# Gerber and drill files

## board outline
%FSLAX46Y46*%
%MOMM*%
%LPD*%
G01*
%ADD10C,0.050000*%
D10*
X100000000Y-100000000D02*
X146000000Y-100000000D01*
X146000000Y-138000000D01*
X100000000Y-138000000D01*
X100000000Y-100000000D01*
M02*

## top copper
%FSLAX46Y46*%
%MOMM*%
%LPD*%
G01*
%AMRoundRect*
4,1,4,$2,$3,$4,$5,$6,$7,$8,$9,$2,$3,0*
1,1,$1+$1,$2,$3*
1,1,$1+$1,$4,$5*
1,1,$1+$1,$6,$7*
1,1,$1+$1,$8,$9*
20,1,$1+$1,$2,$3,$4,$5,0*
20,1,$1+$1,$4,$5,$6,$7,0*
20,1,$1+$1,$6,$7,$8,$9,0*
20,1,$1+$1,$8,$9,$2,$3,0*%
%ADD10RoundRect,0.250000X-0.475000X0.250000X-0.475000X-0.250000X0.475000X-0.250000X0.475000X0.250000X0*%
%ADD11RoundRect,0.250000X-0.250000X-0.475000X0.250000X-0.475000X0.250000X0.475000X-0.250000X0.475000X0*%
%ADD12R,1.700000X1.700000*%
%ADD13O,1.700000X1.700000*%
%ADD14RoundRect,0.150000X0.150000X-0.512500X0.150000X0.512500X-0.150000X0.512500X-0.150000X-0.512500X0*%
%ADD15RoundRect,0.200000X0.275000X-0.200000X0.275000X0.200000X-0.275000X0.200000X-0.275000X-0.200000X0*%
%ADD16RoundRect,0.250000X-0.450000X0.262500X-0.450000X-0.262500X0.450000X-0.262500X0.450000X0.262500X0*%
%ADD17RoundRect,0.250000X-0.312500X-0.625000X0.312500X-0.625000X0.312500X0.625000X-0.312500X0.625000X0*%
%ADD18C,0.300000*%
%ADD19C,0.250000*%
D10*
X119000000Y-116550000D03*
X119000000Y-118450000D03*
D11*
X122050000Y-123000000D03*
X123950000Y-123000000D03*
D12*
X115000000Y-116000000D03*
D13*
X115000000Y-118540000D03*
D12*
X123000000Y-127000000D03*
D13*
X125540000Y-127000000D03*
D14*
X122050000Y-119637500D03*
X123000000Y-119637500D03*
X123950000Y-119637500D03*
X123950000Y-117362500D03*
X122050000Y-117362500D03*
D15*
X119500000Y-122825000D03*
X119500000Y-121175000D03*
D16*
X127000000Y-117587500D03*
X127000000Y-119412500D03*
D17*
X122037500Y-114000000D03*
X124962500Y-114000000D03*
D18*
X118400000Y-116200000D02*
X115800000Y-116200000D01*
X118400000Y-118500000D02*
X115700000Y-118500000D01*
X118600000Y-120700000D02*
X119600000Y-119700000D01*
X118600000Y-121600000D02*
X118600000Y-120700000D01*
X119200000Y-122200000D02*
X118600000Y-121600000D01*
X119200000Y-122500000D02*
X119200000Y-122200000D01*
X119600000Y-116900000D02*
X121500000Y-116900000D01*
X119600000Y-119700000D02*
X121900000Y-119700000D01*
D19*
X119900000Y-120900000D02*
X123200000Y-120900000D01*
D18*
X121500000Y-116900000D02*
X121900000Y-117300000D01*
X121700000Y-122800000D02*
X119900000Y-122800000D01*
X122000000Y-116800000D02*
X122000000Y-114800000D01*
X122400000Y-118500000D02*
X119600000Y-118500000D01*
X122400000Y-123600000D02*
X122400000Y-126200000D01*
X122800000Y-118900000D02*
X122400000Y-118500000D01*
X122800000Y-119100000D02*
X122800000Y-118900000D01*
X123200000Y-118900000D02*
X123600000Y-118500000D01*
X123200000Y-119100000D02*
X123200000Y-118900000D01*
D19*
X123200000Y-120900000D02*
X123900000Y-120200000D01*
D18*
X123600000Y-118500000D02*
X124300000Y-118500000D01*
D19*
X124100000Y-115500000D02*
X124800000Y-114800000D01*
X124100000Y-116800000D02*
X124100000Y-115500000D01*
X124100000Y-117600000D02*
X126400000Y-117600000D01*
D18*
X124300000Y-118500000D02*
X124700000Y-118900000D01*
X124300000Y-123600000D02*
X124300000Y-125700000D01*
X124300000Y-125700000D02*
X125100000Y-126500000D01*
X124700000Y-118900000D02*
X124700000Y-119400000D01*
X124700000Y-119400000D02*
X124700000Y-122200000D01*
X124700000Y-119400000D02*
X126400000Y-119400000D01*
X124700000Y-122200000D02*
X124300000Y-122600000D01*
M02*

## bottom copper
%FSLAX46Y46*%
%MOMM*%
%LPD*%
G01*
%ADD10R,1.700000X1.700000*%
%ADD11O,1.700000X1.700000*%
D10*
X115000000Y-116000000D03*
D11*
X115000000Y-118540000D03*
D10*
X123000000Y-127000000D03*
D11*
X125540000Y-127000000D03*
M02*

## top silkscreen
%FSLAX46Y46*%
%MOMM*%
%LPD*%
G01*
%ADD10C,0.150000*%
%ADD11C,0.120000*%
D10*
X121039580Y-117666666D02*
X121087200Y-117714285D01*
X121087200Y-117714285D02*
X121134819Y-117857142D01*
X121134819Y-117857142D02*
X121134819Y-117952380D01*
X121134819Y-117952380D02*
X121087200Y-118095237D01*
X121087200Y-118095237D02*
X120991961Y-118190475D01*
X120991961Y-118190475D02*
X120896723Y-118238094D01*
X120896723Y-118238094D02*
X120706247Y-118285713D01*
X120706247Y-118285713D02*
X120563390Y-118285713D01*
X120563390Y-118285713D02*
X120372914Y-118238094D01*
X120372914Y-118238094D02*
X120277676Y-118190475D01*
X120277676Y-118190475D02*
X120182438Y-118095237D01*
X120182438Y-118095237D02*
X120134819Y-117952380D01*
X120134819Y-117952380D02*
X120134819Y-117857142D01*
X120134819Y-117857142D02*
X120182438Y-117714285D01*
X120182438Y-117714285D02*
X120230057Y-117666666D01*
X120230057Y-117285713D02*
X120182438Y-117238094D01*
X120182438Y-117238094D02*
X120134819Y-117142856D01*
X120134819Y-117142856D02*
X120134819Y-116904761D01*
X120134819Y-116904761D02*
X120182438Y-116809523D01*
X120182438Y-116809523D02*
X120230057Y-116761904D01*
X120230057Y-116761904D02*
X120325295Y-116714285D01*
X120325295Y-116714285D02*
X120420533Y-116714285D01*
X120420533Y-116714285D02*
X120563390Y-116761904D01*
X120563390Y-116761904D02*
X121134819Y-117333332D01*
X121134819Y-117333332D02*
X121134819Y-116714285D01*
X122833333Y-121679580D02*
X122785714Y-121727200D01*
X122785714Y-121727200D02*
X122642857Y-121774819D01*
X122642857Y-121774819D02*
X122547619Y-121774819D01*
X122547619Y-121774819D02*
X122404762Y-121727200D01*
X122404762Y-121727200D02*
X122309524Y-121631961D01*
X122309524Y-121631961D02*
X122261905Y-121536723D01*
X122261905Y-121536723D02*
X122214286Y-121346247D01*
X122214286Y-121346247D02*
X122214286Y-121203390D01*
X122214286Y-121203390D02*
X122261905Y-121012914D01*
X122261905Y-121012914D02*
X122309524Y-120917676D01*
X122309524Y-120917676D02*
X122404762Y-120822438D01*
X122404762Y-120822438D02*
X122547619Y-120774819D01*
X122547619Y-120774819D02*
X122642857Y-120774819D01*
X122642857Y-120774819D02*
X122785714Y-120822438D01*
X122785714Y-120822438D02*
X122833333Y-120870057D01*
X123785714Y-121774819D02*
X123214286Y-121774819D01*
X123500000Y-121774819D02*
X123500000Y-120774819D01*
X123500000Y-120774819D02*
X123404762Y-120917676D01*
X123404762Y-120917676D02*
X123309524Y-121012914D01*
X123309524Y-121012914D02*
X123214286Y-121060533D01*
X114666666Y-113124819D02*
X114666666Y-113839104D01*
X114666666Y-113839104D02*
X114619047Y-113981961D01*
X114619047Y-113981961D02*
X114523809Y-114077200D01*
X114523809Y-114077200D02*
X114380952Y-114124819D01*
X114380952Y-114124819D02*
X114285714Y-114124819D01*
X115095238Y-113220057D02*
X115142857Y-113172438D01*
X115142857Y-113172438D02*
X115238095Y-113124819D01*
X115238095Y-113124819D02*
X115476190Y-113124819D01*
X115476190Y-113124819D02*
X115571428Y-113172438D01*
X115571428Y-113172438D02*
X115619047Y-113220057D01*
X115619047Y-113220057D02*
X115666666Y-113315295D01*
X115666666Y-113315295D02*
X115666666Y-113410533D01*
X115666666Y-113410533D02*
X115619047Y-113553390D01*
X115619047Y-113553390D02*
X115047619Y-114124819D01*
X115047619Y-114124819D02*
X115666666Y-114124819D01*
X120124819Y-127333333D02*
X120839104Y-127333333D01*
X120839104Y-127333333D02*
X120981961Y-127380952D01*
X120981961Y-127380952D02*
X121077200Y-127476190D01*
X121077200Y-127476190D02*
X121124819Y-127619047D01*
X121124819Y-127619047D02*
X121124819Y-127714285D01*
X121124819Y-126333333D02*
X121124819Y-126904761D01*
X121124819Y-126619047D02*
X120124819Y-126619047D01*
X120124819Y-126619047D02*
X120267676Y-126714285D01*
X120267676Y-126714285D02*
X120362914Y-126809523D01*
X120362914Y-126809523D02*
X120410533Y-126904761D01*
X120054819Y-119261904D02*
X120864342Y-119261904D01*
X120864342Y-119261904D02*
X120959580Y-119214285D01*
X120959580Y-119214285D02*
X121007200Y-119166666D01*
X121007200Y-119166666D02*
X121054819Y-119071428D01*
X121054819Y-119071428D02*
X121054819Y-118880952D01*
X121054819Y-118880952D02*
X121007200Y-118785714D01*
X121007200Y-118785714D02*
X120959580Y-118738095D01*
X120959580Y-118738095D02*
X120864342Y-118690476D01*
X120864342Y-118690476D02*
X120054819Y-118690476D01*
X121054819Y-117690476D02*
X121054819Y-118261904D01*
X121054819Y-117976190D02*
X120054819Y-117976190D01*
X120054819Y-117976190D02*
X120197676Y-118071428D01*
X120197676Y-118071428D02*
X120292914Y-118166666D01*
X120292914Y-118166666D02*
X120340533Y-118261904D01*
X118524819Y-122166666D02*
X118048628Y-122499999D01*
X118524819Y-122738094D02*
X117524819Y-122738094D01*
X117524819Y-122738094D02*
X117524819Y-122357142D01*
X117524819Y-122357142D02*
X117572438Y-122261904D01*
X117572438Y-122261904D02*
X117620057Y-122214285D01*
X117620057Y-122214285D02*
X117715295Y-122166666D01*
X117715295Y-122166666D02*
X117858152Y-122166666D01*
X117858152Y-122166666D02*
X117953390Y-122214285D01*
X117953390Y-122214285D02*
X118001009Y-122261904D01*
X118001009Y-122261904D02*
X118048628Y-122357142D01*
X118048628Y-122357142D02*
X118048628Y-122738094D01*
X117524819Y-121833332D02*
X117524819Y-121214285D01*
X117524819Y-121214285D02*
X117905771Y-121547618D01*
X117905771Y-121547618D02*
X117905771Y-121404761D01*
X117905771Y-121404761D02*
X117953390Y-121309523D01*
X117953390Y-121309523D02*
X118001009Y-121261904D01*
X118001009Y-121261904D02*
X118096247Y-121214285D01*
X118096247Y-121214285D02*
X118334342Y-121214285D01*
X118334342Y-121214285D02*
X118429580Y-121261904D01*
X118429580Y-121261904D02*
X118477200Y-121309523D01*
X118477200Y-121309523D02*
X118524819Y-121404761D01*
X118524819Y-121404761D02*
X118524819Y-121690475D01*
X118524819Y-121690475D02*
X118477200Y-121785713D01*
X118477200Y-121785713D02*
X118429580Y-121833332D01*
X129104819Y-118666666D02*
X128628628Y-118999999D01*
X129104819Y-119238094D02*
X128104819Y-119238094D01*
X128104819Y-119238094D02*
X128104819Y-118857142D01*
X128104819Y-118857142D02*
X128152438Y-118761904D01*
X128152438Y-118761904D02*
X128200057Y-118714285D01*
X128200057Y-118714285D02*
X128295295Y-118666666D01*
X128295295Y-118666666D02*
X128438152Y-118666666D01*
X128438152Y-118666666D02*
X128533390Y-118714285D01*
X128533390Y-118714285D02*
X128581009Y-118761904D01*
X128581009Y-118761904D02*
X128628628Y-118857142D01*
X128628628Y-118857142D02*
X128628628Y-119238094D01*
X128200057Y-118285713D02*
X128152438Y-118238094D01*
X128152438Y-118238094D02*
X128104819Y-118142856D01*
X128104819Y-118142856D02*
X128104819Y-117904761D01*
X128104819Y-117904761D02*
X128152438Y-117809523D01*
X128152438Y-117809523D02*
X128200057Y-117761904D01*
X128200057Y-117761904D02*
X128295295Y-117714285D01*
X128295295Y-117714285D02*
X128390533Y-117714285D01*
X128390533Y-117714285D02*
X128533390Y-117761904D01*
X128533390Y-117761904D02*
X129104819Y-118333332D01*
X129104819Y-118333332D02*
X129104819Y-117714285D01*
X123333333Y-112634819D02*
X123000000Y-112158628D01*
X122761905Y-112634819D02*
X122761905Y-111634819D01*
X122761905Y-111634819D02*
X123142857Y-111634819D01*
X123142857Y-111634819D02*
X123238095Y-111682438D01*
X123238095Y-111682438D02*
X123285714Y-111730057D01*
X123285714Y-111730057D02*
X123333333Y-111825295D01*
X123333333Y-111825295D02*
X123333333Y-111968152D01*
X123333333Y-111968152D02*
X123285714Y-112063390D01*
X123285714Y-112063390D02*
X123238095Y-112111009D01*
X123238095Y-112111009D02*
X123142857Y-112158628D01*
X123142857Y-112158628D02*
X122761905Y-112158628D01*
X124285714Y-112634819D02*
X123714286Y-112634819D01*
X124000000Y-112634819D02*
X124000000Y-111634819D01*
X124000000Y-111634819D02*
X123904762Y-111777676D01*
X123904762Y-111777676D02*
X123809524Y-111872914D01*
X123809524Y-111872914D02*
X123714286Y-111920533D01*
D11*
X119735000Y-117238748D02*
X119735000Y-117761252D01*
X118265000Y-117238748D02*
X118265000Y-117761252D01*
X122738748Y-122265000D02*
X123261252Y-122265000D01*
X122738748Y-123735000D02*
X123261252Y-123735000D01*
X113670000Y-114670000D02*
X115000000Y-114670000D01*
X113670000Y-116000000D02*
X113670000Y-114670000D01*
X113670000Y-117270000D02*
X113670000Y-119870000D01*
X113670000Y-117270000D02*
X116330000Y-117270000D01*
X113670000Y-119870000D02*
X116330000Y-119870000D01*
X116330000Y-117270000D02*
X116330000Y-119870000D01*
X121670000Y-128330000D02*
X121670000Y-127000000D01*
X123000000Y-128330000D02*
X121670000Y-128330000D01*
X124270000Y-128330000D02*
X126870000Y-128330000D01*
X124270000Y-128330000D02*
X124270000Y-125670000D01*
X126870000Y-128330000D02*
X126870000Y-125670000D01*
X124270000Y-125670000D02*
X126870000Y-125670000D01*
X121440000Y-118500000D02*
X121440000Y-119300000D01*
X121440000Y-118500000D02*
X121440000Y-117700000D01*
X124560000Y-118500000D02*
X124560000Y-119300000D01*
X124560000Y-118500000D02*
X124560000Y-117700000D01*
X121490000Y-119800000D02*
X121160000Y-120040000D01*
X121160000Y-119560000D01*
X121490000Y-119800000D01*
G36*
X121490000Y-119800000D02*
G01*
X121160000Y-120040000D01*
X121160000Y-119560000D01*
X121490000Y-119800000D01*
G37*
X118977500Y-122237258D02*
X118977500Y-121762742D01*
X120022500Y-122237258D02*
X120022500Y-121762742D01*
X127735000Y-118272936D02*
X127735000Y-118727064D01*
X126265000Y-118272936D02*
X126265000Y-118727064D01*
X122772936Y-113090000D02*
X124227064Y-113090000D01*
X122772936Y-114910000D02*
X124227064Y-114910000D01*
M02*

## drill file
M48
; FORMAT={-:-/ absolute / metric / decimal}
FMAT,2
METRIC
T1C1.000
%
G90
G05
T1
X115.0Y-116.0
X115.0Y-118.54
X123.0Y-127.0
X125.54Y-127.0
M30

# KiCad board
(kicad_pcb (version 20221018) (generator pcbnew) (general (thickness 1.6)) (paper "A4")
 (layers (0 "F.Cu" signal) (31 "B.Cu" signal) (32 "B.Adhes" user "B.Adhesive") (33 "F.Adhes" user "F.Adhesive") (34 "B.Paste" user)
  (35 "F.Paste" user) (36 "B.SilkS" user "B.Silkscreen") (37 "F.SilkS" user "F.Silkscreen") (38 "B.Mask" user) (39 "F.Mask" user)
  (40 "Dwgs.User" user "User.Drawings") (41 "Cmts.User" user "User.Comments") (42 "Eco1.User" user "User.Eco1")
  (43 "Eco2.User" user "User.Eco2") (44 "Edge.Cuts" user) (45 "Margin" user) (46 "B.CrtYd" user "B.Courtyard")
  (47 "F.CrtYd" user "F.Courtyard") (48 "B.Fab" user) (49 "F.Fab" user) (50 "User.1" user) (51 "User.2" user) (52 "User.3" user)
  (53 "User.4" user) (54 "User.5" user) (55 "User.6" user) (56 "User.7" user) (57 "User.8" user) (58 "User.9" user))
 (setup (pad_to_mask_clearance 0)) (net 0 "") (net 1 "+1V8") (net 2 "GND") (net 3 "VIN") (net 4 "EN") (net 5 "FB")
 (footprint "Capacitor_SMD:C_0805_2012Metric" (layer "F.Cu") (at 119 117.5 -90)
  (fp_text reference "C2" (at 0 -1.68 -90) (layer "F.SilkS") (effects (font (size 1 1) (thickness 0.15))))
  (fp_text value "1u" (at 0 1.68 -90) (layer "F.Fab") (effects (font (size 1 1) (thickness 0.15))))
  (fp_line (start -0.261252 -0.735) (end 0.261252 -0.735) (stroke (width 0.12) (type solid)) (layer "F.SilkS"))
  (fp_line (start -0.261252 0.735) (end 0.261252 0.735) (stroke (width 0.12) (type solid)) (layer "F.SilkS"))
  (pad "1" smd roundrect (at -0.95 0 270) (size 1 1.45) (layers "F.Cu" "F.Paste" "F.Mask") (roundrect_rratio 0.25) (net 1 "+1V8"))
  (pad "2" smd roundrect (at 0.95 0 270) (size 1 1.45) (layers "F.Cu" "F.Paste" "F.Mask") (roundrect_rratio 0.25) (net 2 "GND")))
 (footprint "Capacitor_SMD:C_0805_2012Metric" (layer "F.Cu") (at 123 123)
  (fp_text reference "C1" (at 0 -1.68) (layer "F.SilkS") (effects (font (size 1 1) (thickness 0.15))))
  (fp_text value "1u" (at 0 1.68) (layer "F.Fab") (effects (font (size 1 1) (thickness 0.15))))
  (fp_line (start -0.261252 -0.735) (end 0.261252 -0.735) (stroke (width 0.12) (type solid)) (layer "F.SilkS"))
  (fp_line (start -0.261252 0.735) (end 0.261252 0.735) (stroke (width 0.12) (type solid)) (layer "F.SilkS"))
  (pad "1" smd roundrect (at -0.95 0) (size 1 1.45) (layers "F.Cu" "F.Paste" "F.Mask") (roundrect_rratio 0.25) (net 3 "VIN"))
  (pad "2" smd roundrect (at 0.95 0) (size 1 1.45) (layers "F.Cu" "F.Paste" "F.Mask") (roundrect_rratio 0.25) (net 2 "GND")))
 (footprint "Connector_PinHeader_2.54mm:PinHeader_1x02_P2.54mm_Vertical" (layer "F.Cu") (at 115 116)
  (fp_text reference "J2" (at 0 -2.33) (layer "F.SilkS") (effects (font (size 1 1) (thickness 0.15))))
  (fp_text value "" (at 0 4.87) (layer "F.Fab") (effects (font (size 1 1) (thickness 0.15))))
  (fp_line (start -1.33 -1.33) (end 0 -1.33) (stroke (width 0.12) (type solid)) (layer "F.SilkS"))
  (fp_line (start -1.33 0) (end -1.33 -1.33) (stroke (width 0.12) (type solid)) (layer "F.SilkS"))
  (fp_line (start -1.33 1.27) (end -1.33 3.87) (stroke (width 0.12) (type solid)) (layer "F.SilkS"))
  (fp_line (start -1.33 1.27) (end 1.33 1.27) (stroke (width 0.12) (type solid)) (layer "F.SilkS"))
  (fp_line (start -1.33 3.87) (end 1.33 3.87) (stroke (width 0.12) (type solid)) (layer "F.SilkS"))
  (fp_line (start 1.33 1.27) (end 1.33 3.87) (stroke (width 0.12) (type solid)) (layer "F.SilkS"))
  (pad "1" thru_hole rect (at 0 0) (size 1.7 1.7) (drill 1) (layers "*.Cu" "*.Mask") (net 1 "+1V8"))
  (pad "2" thru_hole oval (at 0 2.54) (size 1.7 1.7) (drill 1) (layers "*.Cu" "*.Mask") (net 2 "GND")))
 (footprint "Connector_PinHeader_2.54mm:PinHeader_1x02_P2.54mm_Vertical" (layer "F.Cu") (at 123 127 90)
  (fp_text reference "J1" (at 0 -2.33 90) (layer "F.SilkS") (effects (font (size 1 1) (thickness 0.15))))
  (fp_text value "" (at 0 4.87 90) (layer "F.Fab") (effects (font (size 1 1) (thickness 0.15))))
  (fp_line (start -1.33 -1.33) (end 0 -1.33) (stroke (width 0.12) (type solid)) (layer "F.SilkS"))
  (fp_line (start -1.33 0) (end -1.33 -1.33) (stroke (width 0.12) (type solid)) (layer "F.SilkS"))
  (fp_line (start -1.33 1.27) (end -1.33 3.87) (stroke (width 0.12) (type solid)) (layer "F.SilkS"))
  (fp_line (start -1.33 1.27) (end 1.33 1.27) (stroke (width 0.12) (type solid)) (layer "F.SilkS"))
  (fp_line (start -1.33 3.87) (end 1.33 3.87) (stroke (width 0.12) (type solid)) (layer "F.SilkS"))
  (fp_line (start 1.33 1.27) (end 1.33 3.87) (stroke (width 0.12) (type solid)) (layer "F.SilkS"))
  (pad "1" thru_hole rect (at 0 0 90) (size 1.7 1.7) (drill 1) (layers "*.Cu" "*.Mask") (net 3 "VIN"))
  (pad "2" thru_hole oval (at 0 2.54 90) (size 1.7 1.7) (drill 1) (layers "*.Cu" "*.Mask") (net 2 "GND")))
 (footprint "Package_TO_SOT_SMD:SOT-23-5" (layer "F.Cu") (at 123 118.5 90)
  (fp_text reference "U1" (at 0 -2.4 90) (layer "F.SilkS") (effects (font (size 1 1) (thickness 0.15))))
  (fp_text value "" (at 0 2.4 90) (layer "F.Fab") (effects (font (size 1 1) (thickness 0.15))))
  (fp_line (start 0 -1.56) (end -0.8 -1.56) (stroke (width 0.12) (type solid)) (layer "F.SilkS"))
  (fp_line (start 0 -1.56) (end 0.8 -1.56) (stroke (width 0.12) (type solid)) (layer "F.SilkS"))
  (fp_line (start 0 1.56) (end -0.8 1.56) (stroke (width 0.12) (type solid)) (layer "F.SilkS"))
  (fp_line (start 0 1.56) (end 0.8 1.56) (stroke (width 0.12) (type solid)) (layer "F.SilkS"))
  (fp_poly
   (pts (xy -1.3 -1.51) (xy -1.54 -1.84) (xy -1.06 -1.84) (xy -1.3 -1.51)) (stroke (width 0.12) (type solid)) (fill solid) (layer "F.SilkS"))
  (pad "1" smd roundrect (at -1.1375 -0.95 90) (size 1.325 0.6) (layers "F.Cu" "F.Paste" "F.Mask") (roundrect_rratio 0.25) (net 3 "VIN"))
  (pad "2" smd roundrect (at -1.1375 0 90) (size 1.325 0.6) (layers "F.Cu" "F.Paste" "F.Mask") (roundrect_rratio 0.25) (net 2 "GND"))
  (pad "3" smd roundrect (at -1.1375 0.95 90) (size 1.325 0.6) (layers "F.Cu" "F.Paste" "F.Mask") (roundrect_rratio 0.25) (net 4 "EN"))
  (pad "4" smd roundrect (at 1.1375 0.95 90) (size 1.325 0.6) (layers "F.Cu" "F.Paste" "F.Mask") (roundrect_rratio 0.25) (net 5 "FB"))
  (pad "5" smd roundrect (at 1.1375 -0.95 90) (size 1.325 0.6) (layers "F.Cu" "F.Paste" "F.Mask") (roundrect_rratio 0.25) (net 1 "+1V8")))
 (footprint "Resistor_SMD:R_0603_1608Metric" (layer "F.Cu") (at 119.5 122 90)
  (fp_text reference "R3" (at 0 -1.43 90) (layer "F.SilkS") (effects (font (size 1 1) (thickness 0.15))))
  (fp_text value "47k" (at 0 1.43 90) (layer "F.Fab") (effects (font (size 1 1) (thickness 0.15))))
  (fp_line (start -0.237258 -0.5225) (end 0.237258 -0.5225) (stroke (width 0.12) (type solid)) (layer "F.SilkS"))
  (fp_line (start -0.237258 0.5225) (end 0.237258 0.5225) (stroke (width 0.12) (type solid)) (layer "F.SilkS"))
  (pad "1" smd roundrect (at -0.825 0 90) (size 0.8 0.95) (layers "F.Cu" "F.Paste" "F.Mask") (roundrect_rratio 0.25) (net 3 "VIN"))
  (pad "2" smd roundrect (at 0.825 0 90) (size 0.8 0.95) (layers "F.Cu" "F.Paste" "F.Mask") (roundrect_rratio 0.25) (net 4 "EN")))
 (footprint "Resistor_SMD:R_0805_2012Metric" (layer "F.Cu") (at 127 118.5 -90)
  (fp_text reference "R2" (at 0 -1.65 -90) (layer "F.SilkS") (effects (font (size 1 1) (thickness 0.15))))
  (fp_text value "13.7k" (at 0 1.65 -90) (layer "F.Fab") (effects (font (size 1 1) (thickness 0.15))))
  (fp_line (start -0.227064 -0.735) (end 0.227064 -0.735) (stroke (width 0.12) (type solid)) (layer "F.SilkS"))
  (fp_line (start -0.227064 0.735) (end 0.227064 0.735) (stroke (width 0.12) (type solid)) (layer "F.SilkS"))
  (pad "1" smd roundrect (at -0.9125 0 270) (size 1.025 1.4) (layers "F.Cu" "F.Paste" "F.Mask") (roundrect_rratio 0.243902) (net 5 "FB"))
  (pad "2" smd roundrect (at 0.9125 0 270) (size 1.025 1.4) (layers "F.Cu" "F.Paste" "F.Mask") (roundrect_rratio 0.243902) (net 2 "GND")))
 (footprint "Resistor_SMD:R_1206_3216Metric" (layer "F.Cu") (at 123.5 114)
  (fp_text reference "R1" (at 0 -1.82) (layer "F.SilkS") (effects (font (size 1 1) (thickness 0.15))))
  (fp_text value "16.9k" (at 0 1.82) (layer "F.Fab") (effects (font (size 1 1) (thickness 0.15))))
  (fp_line (start -0.727064 -0.91) (end 0.727064 -0.91) (stroke (width 0.12) (type solid)) (layer "F.SilkS"))
  (fp_line (start -0.727064 0.91) (end 0.727064 0.91) (stroke (width 0.12) (type solid)) (layer "F.SilkS"))
  (pad "1" smd roundrect (at -1.4625 0) (size 1.125 1.75) (layers "F.Cu" "F.Paste" "F.Mask") (roundrect_rratio 0.222222) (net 1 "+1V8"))
  (pad "2" smd roundrect (at 1.4625 0) (size 1.125 1.75) (layers "F.Cu" "F.Paste" "F.Mask") (roundrect_rratio 0.222222) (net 5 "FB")))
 (gr_rect (start 100 100) (end 146 138) (stroke (width 0.05) (type default)) (fill none) (layer "Edge.Cuts"))
 (segment (start 118.4 116.2) (end 115.8 116.2) (width 0.3) (layer "F.Cu") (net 1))
 (segment (start 118.4 118.5) (end 115.7 118.5) (width 0.3) (layer "F.Cu") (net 2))
 (segment (start 118.6 120.7) (end 119.6 119.7) (width 0.3) (layer "F.Cu") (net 3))
 (segment (start 118.6 121.6) (end 118.6 120.7) (width 0.3) (layer "F.Cu") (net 3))
 (segment (start 119.2 122.2) (end 118.6 121.6) (width 0.3) (layer "F.Cu") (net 3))
 (segment (start 119.2 122.5) (end 119.2 122.2) (width 0.3) (layer "F.Cu") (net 3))
 (segment (start 119.6 116.9) (end 121.5 116.9) (width 0.3) (layer "F.Cu") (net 1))
 (segment (start 119.6 119.7) (end 121.9 119.7) (width 0.3) (layer "F.Cu") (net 3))
 (segment (start 119.9 120.9) (end 123.2 120.9) (width 0.25) (layer "F.Cu") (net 4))
 (segment (start 121.5 116.9) (end 121.9 117.3) (width 0.3) (layer "F.Cu") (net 1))
 (segment (start 121.7 122.8) (end 119.9 122.8) (width 0.3) (layer "F.Cu") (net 3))
 (segment (start 122 116.8) (end 122 114.8) (width 0.3) (layer "F.Cu") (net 1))
 (segment (start 122.4 118.5) (end 119.6 118.5) (width 0.3) (layer "F.Cu") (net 2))
 (segment (start 122.4 123.6) (end 122.4 126.2) (width 0.3) (layer "F.Cu") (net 3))
 (segment (start 122.8 118.9) (end 122.4 118.5) (width 0.3) (layer "F.Cu") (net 2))
 (segment (start 122.8 119.1) (end 122.8 118.9) (width 0.3) (layer "F.Cu") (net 2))
 (segment (start 123.2 118.9) (end 123.6 118.5) (width 0.3) (layer "F.Cu") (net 2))
 (segment (start 123.2 119.1) (end 123.2 118.9) (width 0.3) (layer "F.Cu") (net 2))
 (segment (start 123.2 120.9) (end 123.9 120.2) (width 0.25) (layer "F.Cu") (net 4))
 (segment (start 123.6 118.5) (end 124.3 118.5) (width 0.3) (layer "F.Cu") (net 2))
 (segment (start 124.1 115.5) (end 124.8 114.8) (width 0.25) (layer "F.Cu") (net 5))
 (segment (start 124.1 116.8) (end 124.1 115.5) (width 0.25) (layer "F.Cu") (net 5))
 (segment (start 124.1 117.6) (end 126.4 117.6) (width 0.25) (layer "F.Cu") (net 5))
 (segment (start 124.3 118.5) (end 124.7 118.9) (width 0.3) (layer "F.Cu") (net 2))
 (segment (start 124.3 123.6) (end 124.3 125.7) (width 0.3) (layer "F.Cu") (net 2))
 (segment (start 124.3 125.7) (end 125.1 126.5) (width 0.3) (layer "F.Cu") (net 2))
 (segment (start 124.7 118.9) (end 124.7 119.4) (width 0.3) (layer "F.Cu") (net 2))
 (segment (start 124.7 119.4) (end 124.7 122.2) (width 0.3) (layer "F.Cu") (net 2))
 (segment (start 124.7 119.4) (end 126.4 119.4) (width 0.3) (layer "F.Cu") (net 2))
 (segment (start 124.7 122.2) (end 124.3 122.6) (width 0.3) (layer "F.Cu") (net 2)))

